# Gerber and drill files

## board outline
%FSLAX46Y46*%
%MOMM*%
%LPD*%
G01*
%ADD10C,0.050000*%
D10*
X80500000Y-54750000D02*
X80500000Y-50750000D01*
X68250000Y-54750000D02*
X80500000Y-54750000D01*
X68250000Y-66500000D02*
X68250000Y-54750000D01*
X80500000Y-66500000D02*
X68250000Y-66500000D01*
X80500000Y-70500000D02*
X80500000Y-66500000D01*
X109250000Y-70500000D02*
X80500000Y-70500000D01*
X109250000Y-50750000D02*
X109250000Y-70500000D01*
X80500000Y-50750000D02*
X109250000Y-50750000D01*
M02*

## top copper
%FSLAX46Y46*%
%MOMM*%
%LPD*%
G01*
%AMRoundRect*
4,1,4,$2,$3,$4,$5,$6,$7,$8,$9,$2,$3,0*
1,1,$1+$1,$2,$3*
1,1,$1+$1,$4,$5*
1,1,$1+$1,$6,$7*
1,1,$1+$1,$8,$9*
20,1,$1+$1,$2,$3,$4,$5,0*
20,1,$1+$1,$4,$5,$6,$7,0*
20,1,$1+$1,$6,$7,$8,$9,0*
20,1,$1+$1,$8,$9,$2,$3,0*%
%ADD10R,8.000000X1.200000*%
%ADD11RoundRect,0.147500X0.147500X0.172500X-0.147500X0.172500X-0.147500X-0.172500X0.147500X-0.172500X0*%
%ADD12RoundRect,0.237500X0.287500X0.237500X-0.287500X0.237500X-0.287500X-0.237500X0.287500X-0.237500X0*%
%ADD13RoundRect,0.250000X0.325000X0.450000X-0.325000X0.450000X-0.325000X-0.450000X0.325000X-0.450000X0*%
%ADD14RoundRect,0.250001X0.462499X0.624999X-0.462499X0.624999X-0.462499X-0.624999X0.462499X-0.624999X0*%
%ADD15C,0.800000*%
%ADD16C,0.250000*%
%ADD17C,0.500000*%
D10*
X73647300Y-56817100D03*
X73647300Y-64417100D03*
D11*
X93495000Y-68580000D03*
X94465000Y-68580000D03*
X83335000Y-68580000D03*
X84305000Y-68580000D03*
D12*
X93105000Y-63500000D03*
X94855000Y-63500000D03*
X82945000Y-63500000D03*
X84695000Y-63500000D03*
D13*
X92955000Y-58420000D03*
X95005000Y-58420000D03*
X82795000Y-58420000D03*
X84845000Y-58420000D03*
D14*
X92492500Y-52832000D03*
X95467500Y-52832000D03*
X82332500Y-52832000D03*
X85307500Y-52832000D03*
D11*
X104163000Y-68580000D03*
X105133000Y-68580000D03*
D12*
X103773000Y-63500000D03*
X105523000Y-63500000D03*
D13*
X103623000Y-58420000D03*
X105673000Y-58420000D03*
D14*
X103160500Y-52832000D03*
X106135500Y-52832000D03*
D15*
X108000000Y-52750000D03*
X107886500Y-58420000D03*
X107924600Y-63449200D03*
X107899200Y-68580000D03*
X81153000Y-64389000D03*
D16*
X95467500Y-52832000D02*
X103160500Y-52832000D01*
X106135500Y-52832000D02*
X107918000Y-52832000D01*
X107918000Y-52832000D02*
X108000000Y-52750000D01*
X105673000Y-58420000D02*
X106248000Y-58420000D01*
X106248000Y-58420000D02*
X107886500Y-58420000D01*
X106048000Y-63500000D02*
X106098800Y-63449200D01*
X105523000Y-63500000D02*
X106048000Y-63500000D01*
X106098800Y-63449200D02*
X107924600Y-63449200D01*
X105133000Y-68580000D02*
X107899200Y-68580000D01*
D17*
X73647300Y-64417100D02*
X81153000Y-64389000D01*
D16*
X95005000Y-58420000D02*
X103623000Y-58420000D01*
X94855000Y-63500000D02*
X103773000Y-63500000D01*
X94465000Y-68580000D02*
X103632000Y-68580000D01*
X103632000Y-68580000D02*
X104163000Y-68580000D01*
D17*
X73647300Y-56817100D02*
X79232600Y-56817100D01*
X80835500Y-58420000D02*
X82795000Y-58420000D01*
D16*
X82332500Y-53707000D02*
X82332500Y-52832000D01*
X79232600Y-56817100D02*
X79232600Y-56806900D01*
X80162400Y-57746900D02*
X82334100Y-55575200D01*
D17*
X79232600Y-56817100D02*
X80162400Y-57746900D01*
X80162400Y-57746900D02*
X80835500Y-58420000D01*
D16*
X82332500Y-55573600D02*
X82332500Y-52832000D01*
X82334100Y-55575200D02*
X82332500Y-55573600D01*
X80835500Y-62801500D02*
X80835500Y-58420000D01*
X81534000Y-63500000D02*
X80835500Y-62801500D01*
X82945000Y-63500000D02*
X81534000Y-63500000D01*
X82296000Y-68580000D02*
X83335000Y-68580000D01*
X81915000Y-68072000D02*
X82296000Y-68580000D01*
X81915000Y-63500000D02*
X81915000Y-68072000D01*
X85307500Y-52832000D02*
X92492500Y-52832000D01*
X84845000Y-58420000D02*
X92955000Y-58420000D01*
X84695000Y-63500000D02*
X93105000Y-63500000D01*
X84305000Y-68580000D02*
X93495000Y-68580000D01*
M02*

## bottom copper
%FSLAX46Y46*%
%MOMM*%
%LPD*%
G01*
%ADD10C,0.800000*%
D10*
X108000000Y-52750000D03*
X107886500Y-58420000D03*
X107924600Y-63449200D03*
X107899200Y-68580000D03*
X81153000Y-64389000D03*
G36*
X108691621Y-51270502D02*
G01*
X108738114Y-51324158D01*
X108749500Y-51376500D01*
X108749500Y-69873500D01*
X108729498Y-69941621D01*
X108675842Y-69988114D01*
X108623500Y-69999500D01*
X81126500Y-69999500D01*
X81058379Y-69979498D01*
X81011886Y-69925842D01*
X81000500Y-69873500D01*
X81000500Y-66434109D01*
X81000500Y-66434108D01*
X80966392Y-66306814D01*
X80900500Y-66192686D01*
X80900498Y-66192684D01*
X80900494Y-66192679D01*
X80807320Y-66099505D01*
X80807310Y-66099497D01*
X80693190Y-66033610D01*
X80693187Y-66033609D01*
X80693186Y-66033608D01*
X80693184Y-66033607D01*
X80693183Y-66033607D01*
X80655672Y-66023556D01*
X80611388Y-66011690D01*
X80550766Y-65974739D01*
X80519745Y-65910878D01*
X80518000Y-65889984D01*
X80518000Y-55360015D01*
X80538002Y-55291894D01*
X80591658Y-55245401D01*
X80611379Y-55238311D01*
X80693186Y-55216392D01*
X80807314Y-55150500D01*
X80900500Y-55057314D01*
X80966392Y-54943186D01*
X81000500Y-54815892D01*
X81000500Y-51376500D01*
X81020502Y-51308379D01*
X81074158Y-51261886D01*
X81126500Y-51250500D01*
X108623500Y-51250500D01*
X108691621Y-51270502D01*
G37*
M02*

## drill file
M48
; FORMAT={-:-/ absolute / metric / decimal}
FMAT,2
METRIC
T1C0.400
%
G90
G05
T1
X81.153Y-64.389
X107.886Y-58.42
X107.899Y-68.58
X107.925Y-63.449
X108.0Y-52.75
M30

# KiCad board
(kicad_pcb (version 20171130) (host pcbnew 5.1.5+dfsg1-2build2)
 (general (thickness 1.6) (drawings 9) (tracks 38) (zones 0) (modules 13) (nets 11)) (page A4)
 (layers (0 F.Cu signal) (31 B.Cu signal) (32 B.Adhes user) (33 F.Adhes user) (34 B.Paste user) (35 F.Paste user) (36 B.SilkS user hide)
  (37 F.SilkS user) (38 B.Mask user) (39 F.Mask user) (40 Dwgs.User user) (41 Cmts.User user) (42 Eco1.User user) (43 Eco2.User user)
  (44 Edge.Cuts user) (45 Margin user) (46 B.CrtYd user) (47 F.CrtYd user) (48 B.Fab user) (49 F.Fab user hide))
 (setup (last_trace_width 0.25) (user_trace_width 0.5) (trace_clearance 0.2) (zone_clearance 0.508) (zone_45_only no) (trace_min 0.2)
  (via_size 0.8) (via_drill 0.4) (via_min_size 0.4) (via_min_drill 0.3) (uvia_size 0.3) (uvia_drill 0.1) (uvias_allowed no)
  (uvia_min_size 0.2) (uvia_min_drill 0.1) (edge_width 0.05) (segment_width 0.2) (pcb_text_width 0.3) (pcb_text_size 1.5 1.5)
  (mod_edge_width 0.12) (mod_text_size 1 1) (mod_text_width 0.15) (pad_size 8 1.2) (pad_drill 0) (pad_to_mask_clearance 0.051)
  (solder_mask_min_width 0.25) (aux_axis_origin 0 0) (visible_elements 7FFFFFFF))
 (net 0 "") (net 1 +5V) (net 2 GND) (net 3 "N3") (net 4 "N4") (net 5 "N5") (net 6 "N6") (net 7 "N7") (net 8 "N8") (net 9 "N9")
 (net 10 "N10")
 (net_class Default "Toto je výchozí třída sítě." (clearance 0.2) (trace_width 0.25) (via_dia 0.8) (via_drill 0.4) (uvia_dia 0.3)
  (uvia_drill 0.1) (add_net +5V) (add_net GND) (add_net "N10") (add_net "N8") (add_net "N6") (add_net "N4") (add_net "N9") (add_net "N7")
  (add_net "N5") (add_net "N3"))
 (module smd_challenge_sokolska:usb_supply (layer F.Cu) (at 73.6473 60.6171) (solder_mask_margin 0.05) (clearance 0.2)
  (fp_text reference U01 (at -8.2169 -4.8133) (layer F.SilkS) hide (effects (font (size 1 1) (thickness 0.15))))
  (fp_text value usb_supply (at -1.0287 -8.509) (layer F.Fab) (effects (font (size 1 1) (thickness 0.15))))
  (pad VCC smd rect (at 0 -3.8) (size 8 1.2) (layers F.Cu F.Paste F.Mask) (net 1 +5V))
  (pad GND smd rect (at 0 3.8) (size 8 1.2) (layers F.Cu F.Paste F.Mask) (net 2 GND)))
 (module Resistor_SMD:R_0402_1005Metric (layer F.Cu) (at 93.98 68.58 180)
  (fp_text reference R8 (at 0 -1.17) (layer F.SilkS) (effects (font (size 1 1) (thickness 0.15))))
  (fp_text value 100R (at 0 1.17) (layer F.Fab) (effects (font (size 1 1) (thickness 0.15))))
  (pad 2 smd roundrect (at 0.485 0 180) (size 0.59 0.64) (layers F.Cu F.Paste F.Mask) (roundrect_rratio 0.25) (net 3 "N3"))
  (pad 1 smd roundrect (at -0.485 0 180) (size 0.59 0.64) (layers F.Cu F.Paste F.Mask) (roundrect_rratio 0.25) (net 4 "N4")))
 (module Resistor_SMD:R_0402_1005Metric (layer F.Cu) (at 83.82 68.58 180)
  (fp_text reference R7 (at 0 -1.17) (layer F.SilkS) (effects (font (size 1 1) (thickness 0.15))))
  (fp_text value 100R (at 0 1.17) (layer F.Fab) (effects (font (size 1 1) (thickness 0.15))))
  (pad 2 smd roundrect (at 0.485 0 180) (size 0.59 0.64) (layers F.Cu F.Paste F.Mask) (roundrect_rratio 0.25) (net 1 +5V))
  (pad 1 smd roundrect (at -0.485 0 180) (size 0.59 0.64) (layers F.Cu F.Paste F.Mask) (roundrect_rratio 0.25) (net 3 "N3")))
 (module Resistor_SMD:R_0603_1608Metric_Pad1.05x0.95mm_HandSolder (layer F.Cu) (at 93.98 63.5 180)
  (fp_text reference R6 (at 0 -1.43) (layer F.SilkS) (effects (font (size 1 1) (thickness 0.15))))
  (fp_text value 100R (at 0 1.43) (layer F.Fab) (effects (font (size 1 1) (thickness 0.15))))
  (pad 2 smd roundrect (at 0.875 0 180) (size 1.05 0.95) (layers F.Cu F.Paste F.Mask) (roundrect_rratio 0.25) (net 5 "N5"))
  (pad 1 smd roundrect (at -0.875 0 180) (size 1.05 0.95) (layers F.Cu F.Paste F.Mask) (roundrect_rratio 0.25) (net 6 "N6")))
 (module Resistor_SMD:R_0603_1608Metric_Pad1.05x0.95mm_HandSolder (layer F.Cu) (at 83.82 63.5 180)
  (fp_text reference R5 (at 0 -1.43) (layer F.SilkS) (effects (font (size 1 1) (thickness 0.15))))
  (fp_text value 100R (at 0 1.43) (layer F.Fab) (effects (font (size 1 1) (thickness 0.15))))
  (pad 2 smd roundrect (at 0.875 0 180) (size 1.05 0.95) (layers F.Cu F.Paste F.Mask) (roundrect_rratio 0.25) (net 1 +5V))
  (pad 1 smd roundrect (at -0.875 0 180) (size 1.05 0.95) (layers F.Cu F.Paste F.Mask) (roundrect_rratio 0.25) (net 5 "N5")))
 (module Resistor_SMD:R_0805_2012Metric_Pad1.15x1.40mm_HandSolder (layer F.Cu) (at 93.98 58.42 180)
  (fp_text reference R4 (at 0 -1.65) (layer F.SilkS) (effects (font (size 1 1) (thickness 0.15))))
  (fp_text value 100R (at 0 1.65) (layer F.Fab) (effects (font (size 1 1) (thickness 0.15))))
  (pad 2 smd roundrect (at 1.025 0 180) (size 1.15 1.4) (layers F.Cu F.Paste F.Mask) (roundrect_rratio 0.217391) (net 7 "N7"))
  (pad 1 smd roundrect (at -1.025 0 180) (size 1.15 1.4) (layers F.Cu F.Paste F.Mask) (roundrect_rratio 0.217391) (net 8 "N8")))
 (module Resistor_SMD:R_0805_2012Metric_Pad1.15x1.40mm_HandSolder (layer F.Cu) (at 83.82 58.42 180)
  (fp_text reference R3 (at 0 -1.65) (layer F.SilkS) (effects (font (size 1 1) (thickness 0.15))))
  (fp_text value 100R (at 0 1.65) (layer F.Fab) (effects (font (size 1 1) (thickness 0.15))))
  (pad 2 smd roundrect (at 1.025 0 180) (size 1.15 1.4) (layers F.Cu F.Paste F.Mask) (roundrect_rratio 0.217391) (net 1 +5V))
  (pad 1 smd roundrect (at -1.025 0 180) (size 1.15 1.4) (layers F.Cu F.Paste F.Mask) (roundrect_rratio 0.217391) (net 7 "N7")))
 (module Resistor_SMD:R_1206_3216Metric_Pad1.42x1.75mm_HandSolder (layer F.Cu) (at 93.98 52.832 180)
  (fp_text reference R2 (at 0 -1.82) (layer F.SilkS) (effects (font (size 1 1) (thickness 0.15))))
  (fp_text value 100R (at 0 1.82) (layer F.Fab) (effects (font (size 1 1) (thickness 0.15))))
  (pad 2 smd roundrect (at 1.4875 0 180) (size 1.425 1.75) (layers F.Cu F.Paste F.Mask) (roundrect_rratio 0.175439) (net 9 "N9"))
  (pad 1 smd roundrect (at -1.4875 0 180) (size 1.425 1.75) (layers F.Cu F.Paste F.Mask) (roundrect_rratio 0.175439) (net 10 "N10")))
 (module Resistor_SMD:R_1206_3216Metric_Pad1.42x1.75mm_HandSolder (layer F.Cu) (at 83.82 52.832 180)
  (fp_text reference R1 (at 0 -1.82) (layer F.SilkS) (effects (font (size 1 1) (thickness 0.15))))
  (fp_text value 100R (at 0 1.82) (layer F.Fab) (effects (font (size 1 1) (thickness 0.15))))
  (pad 2 smd roundrect (at 1.4875 0 180) (size 1.425 1.75) (layers F.Cu F.Paste F.Mask) (roundrect_rratio 0.175439) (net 1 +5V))
  (pad 1 smd roundrect (at -1.4875 0 180) (size 1.425 1.75) (layers F.Cu F.Paste F.Mask) (roundrect_rratio 0.175439) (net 9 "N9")))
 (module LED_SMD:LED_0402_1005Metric (layer F.Cu) (at 104.648 68.58 180)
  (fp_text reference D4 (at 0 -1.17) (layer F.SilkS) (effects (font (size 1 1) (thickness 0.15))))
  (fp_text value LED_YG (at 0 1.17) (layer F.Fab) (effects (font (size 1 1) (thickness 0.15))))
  (pad 2 smd roundrect (at 0.485 0 180) (size 0.59 0.64) (layers F.Cu F.Paste F.Mask) (roundrect_rratio 0.25) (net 4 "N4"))
  (pad 1 smd roundrect (at -0.485 0 180) (size 0.59 0.64) (layers F.Cu F.Paste F.Mask) (roundrect_rratio 0.25) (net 2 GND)))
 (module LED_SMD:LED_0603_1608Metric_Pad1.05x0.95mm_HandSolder (layer F.Cu) (at 104.648 63.5 180)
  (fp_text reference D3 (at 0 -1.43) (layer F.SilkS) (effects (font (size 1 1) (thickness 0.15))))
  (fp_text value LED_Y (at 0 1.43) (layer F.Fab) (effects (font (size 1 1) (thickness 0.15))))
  (pad 2 smd roundrect (at 0.875 0 180) (size 1.05 0.95) (layers F.Cu F.Paste F.Mask) (roundrect_rratio 0.25) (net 6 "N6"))
  (pad 1 smd roundrect (at -0.875 0 180) (size 1.05 0.95) (layers F.Cu F.Paste F.Mask) (roundrect_rratio 0.25) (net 2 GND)))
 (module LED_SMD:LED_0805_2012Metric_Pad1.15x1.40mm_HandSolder (layer F.Cu) (at 104.648 58.42 180)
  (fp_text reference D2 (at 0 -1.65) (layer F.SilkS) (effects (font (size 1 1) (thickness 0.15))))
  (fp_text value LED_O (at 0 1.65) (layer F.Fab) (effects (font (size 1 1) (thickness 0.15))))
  (pad 2 smd roundrect (at 1.025 0 180) (size 1.15 1.4) (layers F.Cu F.Paste F.Mask) (roundrect_rratio 0.217391) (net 8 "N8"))
  (pad 1 smd roundrect (at -1.025 0 180) (size 1.15 1.4) (layers F.Cu F.Paste F.Mask) (roundrect_rratio 0.217391) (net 2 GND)))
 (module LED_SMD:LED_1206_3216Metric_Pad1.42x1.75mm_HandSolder (layer F.Cu) (at 104.648 52.832 180)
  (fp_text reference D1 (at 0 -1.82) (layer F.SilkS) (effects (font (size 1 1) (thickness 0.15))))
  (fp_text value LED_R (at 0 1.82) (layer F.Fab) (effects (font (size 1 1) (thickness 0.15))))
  (pad 2 smd roundrect (at 1.4875 0 180) (size 1.425 1.75) (layers F.Cu F.Paste F.Mask) (roundrect_rratio 0.175439) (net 10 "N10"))
  (pad 1 smd roundrect (at -1.4875 0 180) (size 1.425 1.75) (layers F.Cu F.Paste F.Mask) (roundrect_rratio 0.175439) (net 2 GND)))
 (gr_line (start 80.5 54.75) (end 80.5 50.75) (layer Edge.Cuts) (width 0.05))
 (gr_line (start 68.25 54.75) (end 80.5 54.75) (layer Edge.Cuts) (width 0.05))
 (gr_line (start 68.25 66.5) (end 68.25 54.75) (layer Edge.Cuts) (width 0.05))
 (gr_line (start 80.5 66.5) (end 68.25 66.5) (layer Edge.Cuts) (width 0.05))
 (gr_line (start 80.5 70.5) (end 80.5 66.5) (layer Edge.Cuts) (width 0.05))
 (gr_line (start 109.25 70.5) (end 80.5 70.5) (layer Edge.Cuts) (width 0.05))
 (gr_line (start 109.25 50.75) (end 109.25 70.5) (layer Edge.Cuts) (width 0.05))
 (gr_line (start 80.5 50.75) (end 109.25 50.75) (layer Edge.Cuts) (width 0.05))
 (segment (start 95.4675 52.832) (end 103.1605 52.832) (width 0.25) (layer F.Cu) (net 10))
 (via (at 108 52.75) (size 0.8) (drill 0.4) (layers F.Cu B.Cu) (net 2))
 (segment (start 106.1355 52.832) (end 107.918 52.832) (width 0.25) (layer F.Cu) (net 2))
 (segment (start 107.918 52.832) (end 108 52.75) (width 0.25) (layer F.Cu) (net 2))
 (segment (start 105.673 58.42) (end 106.248 58.42) (width 0.25) (layer F.Cu) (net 2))
 (via (at 107.8865 58.42) (size 0.8) (drill 0.4) (layers F.Cu B.Cu) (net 2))
 (segment (start 106.248 58.42) (end 107.8865 58.42) (width 0.25) (layer F.Cu) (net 2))
 (segment (start 106.048 63.5) (end 106.0988 63.4492) (width 0.25) (layer F.Cu) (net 2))
 (segment (start 105.523 63.5) (end 106.048 63.5) (width 0.25) (layer F.Cu) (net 2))
 (via (at 107.9246 63.4492) (size 0.8) (drill 0.4) (layers F.Cu B.Cu) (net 2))
 (segment (start 106.0988 63.4492) (end 107.9246 63.4492) (width 0.25) (layer F.Cu) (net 2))
 (via (at 107.8992 68.58) (size 0.8) (drill 0.4) (layers F.Cu B.Cu) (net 2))
 (segment (start 105.133 68.58) (end 107.8992 68.58) (width 0.25) (layer F.Cu) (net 2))
 (segment (start 73.6473 64.4171) (end 81.153 64.389) (width 0.5) (layer F.Cu) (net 2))
 (via (at 81.153 64.389) (size 0.8) (drill 0.4) (layers F.Cu B.Cu) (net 2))
 (segment (start 95.005 58.42) (end 103.623 58.42) (width 0.25) (layer F.Cu) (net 8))
 (segment (start 94.855 63.5) (end 103.773 63.5) (width 0.25) (layer F.Cu) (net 6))
 (segment (start 94.465 68.58) (end 103.632 68.58) (width 0.25) (layer F.Cu) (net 4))
 (segment (start 103.632 68.58) (end 104.163 68.58) (width 0.25) (layer F.Cu) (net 4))
 (segment (start 73.6473 56.8171) (end 79.2326 56.8171) (width 0.5) (layer F.Cu) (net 1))
 (segment (start 80.8355 58.42) (end 82.795 58.42) (width 0.5) (layer F.Cu) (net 1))
 (segment (start 82.3325 53.707) (end 82.3325 52.832) (width 0.25) (layer F.Cu) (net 1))
 (segment (start 79.2326 56.8171) (end 79.2326 56.8069) (width 0.25) (layer F.Cu) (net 1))
 (segment (start 80.1624 57.7469) (end 82.3341 55.5752) (width 0.25) (layer F.Cu) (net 1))
 (segment (start 79.2326 56.8171) (end 80.1624 57.7469) (width 0.5) (layer F.Cu) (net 1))
 (segment (start 80.1624 57.7469) (end 80.8355 58.42) (width 0.5) (layer F.Cu) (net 1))
 (segment (start 82.3325 55.5736) (end 82.3325 52.832) (width 0.25) (layer F.Cu) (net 1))
 (segment (start 82.3341 55.5752) (end 82.3325 55.5736) (width 0.25) (layer F.Cu) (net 1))
 (segment (start 80.8355 62.8015) (end 80.8355 58.42) (width 0.25) (layer F.Cu) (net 1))
 (segment (start 81.534 63.5) (end 80.8355 62.8015) (width 0.25) (layer F.Cu) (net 1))
 (segment (start 82.945 63.5) (end 81.534 63.5) (width 0.25) (layer F.Cu) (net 1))
 (segment (start 82.296 68.58) (end 83.335 68.58) (width 0.25) (layer F.Cu) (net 1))
 (segment (start 81.915 68.072) (end 82.296 68.58) (width 0.25) (layer F.Cu) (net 1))
 (segment (start 81.915 63.5) (end 81.915 68.072) (width 0.25) (layer F.Cu) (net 1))
 (segment (start 85.3075 52.832) (end 92.4925 52.832) (width 0.25) (layer F.Cu) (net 9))
 (segment (start 84.845 58.42) (end 92.955 58.42) (width 0.25) (layer F.Cu) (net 7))
 (segment (start 84.695 63.5) (end 93.105 63.5) (width 0.25) (layer F.Cu) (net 5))
 (segment (start 84.305 68.58) (end 93.495 68.58) (width 0.25) (layer F.Cu) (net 3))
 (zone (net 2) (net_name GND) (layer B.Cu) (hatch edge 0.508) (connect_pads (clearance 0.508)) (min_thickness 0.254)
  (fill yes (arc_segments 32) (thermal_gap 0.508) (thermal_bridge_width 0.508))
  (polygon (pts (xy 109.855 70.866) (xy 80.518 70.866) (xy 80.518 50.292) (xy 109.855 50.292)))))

